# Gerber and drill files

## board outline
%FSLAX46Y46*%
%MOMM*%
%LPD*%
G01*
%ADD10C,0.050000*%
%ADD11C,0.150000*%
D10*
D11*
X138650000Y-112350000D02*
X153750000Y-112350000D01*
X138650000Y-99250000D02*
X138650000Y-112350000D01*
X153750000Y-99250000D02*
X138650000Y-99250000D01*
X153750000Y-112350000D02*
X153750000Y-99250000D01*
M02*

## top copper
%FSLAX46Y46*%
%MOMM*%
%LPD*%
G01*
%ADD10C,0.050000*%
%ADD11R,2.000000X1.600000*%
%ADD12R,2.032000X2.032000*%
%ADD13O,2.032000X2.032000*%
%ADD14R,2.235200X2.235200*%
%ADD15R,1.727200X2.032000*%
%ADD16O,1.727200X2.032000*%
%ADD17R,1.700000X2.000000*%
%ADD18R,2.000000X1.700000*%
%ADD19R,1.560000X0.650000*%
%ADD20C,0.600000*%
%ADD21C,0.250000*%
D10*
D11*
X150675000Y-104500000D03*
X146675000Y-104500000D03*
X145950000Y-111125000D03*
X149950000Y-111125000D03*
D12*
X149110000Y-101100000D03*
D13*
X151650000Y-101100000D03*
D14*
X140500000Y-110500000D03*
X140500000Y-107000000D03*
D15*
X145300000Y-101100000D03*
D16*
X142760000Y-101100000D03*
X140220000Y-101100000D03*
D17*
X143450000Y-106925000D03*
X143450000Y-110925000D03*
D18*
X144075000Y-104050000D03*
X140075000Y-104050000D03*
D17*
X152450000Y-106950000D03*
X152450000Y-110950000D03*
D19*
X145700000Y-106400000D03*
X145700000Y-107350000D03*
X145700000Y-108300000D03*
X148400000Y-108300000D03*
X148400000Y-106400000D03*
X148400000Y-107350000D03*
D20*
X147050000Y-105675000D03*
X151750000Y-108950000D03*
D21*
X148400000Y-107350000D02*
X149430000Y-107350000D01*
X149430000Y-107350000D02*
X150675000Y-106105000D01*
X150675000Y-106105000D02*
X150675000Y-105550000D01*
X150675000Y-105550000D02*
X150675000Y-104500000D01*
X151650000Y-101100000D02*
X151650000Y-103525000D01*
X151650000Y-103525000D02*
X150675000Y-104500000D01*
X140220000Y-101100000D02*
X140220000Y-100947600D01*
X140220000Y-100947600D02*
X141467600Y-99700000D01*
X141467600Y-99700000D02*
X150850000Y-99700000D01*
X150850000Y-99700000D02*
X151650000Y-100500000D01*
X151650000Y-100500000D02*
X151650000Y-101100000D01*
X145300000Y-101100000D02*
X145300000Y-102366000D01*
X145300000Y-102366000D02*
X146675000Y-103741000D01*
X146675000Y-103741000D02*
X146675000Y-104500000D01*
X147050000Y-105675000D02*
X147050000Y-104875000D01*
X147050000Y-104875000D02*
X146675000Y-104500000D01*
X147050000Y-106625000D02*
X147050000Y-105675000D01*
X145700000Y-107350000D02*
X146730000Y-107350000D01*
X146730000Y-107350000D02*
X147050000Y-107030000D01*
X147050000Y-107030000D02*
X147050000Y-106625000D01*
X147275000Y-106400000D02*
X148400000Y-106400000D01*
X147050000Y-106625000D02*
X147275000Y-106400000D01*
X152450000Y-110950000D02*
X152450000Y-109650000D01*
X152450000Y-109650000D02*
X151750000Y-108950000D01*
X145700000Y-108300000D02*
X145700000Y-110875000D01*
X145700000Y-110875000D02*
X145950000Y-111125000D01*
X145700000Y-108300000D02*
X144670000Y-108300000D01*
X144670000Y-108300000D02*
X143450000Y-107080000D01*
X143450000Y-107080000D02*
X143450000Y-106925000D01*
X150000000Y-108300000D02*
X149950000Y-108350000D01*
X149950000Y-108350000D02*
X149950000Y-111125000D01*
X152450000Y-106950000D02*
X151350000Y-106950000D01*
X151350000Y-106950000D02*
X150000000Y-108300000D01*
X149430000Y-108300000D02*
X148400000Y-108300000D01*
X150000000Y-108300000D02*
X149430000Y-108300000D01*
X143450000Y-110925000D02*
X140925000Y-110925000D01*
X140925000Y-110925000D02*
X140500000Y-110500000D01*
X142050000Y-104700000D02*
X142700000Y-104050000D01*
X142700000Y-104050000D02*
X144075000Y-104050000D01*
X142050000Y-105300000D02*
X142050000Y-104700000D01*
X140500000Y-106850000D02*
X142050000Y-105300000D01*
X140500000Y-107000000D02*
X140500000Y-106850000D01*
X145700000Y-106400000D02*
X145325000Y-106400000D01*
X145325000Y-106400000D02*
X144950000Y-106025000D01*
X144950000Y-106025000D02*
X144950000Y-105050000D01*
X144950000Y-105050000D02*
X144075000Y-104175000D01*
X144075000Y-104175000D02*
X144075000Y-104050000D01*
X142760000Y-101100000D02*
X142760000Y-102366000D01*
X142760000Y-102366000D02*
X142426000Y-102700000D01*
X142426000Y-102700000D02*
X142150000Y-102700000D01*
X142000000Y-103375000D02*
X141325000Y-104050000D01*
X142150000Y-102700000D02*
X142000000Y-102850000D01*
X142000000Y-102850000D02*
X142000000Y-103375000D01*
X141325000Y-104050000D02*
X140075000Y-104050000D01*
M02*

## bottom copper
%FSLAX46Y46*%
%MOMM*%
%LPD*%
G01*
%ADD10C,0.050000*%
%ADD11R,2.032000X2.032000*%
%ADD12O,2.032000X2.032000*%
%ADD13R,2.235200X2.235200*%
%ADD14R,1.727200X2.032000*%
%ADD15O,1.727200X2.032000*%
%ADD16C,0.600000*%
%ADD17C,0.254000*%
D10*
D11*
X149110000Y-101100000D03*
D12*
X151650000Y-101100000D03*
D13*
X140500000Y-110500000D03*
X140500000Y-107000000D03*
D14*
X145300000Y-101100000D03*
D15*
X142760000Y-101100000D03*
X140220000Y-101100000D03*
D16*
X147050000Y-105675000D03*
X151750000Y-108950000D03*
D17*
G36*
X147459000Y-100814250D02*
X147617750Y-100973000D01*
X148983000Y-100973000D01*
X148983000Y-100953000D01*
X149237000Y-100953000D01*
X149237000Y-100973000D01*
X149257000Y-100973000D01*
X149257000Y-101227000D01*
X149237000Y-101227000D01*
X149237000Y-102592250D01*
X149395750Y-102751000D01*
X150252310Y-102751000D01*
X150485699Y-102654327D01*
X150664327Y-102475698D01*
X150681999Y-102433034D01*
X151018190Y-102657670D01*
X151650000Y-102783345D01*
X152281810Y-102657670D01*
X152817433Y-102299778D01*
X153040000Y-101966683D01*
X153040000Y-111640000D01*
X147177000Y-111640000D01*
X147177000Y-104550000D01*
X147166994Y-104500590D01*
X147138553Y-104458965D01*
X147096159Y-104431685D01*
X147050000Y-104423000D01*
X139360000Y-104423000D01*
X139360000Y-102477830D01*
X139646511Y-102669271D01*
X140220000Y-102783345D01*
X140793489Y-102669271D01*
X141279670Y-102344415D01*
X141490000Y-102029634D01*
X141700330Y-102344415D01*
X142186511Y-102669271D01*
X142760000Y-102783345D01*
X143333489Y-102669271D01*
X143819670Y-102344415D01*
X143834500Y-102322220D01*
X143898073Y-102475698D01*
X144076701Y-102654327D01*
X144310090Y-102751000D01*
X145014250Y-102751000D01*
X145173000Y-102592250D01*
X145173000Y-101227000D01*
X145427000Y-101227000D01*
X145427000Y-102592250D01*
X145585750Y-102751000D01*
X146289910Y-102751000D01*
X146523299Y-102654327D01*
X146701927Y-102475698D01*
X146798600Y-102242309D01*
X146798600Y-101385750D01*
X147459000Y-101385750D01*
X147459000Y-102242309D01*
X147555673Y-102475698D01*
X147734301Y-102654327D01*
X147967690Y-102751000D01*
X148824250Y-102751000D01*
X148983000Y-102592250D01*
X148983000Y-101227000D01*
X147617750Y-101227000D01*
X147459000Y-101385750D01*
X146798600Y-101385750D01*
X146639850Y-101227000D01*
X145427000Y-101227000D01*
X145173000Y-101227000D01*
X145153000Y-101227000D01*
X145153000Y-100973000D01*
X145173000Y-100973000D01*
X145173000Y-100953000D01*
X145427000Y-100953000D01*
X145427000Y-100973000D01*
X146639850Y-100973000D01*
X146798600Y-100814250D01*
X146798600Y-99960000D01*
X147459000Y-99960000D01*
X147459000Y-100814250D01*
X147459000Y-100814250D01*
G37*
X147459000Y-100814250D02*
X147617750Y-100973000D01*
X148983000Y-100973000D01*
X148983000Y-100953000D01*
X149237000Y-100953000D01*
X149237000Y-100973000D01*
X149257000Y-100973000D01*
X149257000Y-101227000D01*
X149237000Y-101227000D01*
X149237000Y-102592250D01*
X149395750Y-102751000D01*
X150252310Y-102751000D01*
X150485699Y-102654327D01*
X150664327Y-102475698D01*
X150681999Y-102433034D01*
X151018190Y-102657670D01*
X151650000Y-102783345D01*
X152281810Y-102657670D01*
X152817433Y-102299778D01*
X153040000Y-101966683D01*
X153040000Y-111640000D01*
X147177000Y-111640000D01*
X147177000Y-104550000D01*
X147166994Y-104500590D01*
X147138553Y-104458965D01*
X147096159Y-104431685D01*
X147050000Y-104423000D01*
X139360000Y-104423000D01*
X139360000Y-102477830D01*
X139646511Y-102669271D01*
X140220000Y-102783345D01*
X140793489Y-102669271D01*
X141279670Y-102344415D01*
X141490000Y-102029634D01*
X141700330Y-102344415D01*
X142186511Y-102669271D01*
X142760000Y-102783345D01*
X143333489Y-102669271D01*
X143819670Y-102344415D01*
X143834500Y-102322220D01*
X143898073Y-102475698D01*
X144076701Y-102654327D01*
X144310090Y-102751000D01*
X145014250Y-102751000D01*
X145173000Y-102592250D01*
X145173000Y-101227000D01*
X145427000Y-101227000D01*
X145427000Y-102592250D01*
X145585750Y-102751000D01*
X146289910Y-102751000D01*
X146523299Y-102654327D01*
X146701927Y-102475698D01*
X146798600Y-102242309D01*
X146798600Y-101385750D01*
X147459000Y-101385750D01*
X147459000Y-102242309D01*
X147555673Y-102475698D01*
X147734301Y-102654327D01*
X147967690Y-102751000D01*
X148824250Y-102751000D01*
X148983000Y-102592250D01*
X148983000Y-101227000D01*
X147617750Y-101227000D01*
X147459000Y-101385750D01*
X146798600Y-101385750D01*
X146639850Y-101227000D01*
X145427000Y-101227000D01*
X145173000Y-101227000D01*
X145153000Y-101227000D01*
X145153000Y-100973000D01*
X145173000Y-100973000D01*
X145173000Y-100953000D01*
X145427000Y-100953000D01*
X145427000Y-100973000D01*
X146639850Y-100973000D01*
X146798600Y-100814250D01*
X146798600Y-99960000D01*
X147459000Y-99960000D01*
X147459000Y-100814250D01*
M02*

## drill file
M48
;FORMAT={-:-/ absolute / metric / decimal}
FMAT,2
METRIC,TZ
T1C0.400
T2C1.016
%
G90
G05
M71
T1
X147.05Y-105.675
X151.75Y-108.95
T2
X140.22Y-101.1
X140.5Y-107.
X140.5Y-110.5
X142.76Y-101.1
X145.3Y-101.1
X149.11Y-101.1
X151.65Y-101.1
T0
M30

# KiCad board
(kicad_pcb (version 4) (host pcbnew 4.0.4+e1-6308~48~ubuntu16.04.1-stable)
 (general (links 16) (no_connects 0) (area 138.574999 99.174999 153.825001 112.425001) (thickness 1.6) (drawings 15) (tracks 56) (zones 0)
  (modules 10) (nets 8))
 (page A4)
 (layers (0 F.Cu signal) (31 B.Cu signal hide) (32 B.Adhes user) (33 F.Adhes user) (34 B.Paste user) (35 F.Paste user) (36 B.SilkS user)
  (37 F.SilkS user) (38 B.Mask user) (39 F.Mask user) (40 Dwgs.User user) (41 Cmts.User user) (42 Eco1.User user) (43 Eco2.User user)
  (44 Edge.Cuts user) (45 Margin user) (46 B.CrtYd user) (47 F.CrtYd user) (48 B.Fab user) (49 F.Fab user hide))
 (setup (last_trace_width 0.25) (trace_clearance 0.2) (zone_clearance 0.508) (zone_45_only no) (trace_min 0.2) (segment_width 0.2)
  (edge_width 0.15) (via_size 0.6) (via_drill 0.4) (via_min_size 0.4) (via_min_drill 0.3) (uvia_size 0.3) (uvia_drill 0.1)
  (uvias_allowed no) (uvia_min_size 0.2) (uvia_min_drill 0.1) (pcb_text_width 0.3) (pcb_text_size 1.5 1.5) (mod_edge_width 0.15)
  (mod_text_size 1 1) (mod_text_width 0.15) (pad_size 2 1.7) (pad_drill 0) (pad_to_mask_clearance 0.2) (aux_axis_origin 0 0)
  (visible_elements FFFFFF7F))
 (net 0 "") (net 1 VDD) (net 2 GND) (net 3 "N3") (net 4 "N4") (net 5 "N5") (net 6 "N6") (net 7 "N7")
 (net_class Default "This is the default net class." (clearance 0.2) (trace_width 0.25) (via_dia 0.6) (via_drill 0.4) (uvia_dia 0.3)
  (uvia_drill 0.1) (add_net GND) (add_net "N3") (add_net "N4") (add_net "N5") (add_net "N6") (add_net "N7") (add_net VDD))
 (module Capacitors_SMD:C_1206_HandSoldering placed (layer F.Cu) (at 148.675 104.5 180)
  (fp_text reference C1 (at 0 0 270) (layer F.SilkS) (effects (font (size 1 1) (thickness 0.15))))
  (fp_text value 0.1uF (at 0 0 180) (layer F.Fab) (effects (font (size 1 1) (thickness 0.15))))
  (pad 1 smd rect (at -2 0 180) (size 2 1.6) (layers F.Cu F.Paste F.Mask) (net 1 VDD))
  (pad 2 smd rect (at 2 0 180) (size 2 1.6) (layers F.Cu F.Paste F.Mask) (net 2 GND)))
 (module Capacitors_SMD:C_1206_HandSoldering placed (layer F.Cu) (at 147.95 111.125)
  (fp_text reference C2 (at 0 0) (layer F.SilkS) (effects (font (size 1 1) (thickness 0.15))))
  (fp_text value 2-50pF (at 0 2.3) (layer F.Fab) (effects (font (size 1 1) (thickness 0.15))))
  (pad 1 smd rect (at -2 0) (size 2 1.6) (layers F.Cu F.Paste F.Mask) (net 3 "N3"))
  (pad 2 smd rect (at 2 0) (size 2 1.6) (layers F.Cu F.Paste F.Mask) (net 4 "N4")))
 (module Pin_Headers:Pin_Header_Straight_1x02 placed (layer F.Cu) (at 149.11 101.1 90)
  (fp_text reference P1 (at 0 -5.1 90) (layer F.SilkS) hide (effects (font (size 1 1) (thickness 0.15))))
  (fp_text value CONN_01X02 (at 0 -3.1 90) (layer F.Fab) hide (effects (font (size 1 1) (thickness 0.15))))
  (pad 1 thru_hole rect (at 0 0 90) (size 2.032 2.032) (drill 1.016) (layers *.Cu *.Mask F.SilkS) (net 2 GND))
  (pad 2 thru_hole oval (at 0 2.54 90) (size 2.032 2.032) (drill 1.016) (layers *.Cu *.Mask F.SilkS) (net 1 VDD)))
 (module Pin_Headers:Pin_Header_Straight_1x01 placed (layer F.Cu) (at 140.5 110.5 180)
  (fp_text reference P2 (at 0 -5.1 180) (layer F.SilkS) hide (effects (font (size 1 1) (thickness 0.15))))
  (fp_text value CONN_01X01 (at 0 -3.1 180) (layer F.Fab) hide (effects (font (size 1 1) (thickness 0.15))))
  (pad 1 thru_hole rect (at 0 0 180) (size 2.2352 2.2352) (drill 1.016) (layers *.Cu *.Mask F.SilkS) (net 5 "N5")))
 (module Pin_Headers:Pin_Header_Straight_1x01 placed (layer F.Cu) (at 140.5 107 90)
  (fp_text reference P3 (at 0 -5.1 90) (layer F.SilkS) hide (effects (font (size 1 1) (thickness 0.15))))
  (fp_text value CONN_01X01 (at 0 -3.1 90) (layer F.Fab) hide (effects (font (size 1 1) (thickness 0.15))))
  (pad 1 thru_hole rect (at 0 0 90) (size 2.2352 2.2352) (drill 1.016) (layers *.Cu *.Mask F.SilkS) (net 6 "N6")))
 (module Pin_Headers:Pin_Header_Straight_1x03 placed (layer F.Cu) (at 145.3 101.1 270)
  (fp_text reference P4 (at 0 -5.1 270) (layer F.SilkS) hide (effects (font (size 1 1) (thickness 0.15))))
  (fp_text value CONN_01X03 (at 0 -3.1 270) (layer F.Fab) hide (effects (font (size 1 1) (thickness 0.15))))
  (pad 1 thru_hole rect (at 0 0 270) (size 2.032 1.7272) (drill 1.016) (layers *.Cu *.Mask F.SilkS) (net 2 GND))
  (pad 2 thru_hole oval (at 0 2.54 270) (size 2.032 1.7272) (drill 1.016) (layers *.Cu *.Mask F.SilkS) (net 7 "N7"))
  (pad 3 thru_hole oval (at 0 5.08 270) (size 2.032 1.7272) (drill 1.016) (layers *.Cu *.Mask F.SilkS) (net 1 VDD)))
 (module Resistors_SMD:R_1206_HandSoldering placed (layer F.Cu) (at 143.45 108.925 270)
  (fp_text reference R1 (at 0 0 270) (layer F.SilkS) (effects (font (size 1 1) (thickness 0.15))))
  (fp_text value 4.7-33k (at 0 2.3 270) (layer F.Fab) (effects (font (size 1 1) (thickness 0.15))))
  (pad 1 smd rect (at -2 0 270) (size 2 1.7) (layers F.Cu F.Paste F.Mask) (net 3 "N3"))
  (pad 2 smd rect (at 2 0 270) (size 2 1.7) (layers F.Cu F.Paste F.Mask) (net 5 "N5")))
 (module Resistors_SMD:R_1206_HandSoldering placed (layer F.Cu) (at 142.075 104.05 180)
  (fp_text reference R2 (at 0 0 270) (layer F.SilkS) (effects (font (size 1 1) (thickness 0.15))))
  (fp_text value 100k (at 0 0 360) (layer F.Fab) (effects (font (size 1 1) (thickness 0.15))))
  (pad 1 smd rect (at -2 0 180) (size 2 1.7) (layers F.Cu F.Paste F.Mask) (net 6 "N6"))
  (pad 2 smd rect (at 2 0 180) (size 2 1.7) (layers F.Cu F.Paste F.Mask) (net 7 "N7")))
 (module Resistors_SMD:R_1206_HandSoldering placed (layer F.Cu) (at 152.45 108.95 270)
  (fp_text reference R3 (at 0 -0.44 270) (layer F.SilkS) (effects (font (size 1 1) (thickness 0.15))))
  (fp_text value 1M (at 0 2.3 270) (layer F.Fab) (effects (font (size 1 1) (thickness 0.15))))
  (pad 1 smd rect (at -2 0 270) (size 2 1.7) (layers F.Cu F.Paste F.Mask) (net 4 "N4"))
  (pad 2 smd rect (at 2 0 270) (size 2 1.7) (layers F.Cu F.Paste F.Mask) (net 2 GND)))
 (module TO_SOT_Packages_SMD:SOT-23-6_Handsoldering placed (layer F.Cu) (at 147.05 107.35)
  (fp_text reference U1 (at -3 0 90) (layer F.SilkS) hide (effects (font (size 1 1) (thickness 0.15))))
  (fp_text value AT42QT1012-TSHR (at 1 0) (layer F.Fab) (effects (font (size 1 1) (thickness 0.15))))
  (pad 1 smd rect (at -1.35 -0.95) (size 1.56 0.65) (layers F.Cu F.Paste F.Mask) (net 6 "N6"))
  (pad 2 smd rect (at -1.35 0) (size 1.56 0.65) (layers F.Cu F.Paste F.Mask) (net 2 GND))
  (pad 3 smd rect (at -1.35 0.95) (size 1.56 0.65) (layers F.Cu F.Paste F.Mask) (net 3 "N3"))
  (pad 4 smd rect (at 1.35 0.95) (size 1.56 0.65) (layers F.Cu F.Paste F.Mask) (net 4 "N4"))
  (pad 6 smd rect (at 1.35 -0.95) (size 1.56 0.65) (layers F.Cu F.Paste F.Mask) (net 2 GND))
  (pad 5 smd rect (at 1.35 0) (size 1.56 0.65) (layers F.Cu F.Paste F.Mask) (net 1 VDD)))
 (gr_line (start 138.65 112.35) (end 153.75 112.35) (layer Edge.Cuts) (width 0.15))
 (gr_line (start 138.65 99.25) (end 138.65 112.35) (layer Edge.Cuts) (width 0.15))
 (gr_line (start 153.75 99.25) (end 138.65 99.25) (layer Edge.Cuts) (width 0.15))
 (gr_line (start 153.75 112.35) (end 153.75 99.25) (layer Edge.Cuts) (width 0.15))
 (segment (start 148.4 107.35) (end 149.43 107.35) (width 0.25) (layer F.Cu) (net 1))
 (segment (start 149.43 107.35) (end 150.675 106.105) (width 0.25) (layer F.Cu) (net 1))
 (segment (start 150.675 106.105) (end 150.675 105.55) (width 0.25) (layer F.Cu) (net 1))
 (segment (start 150.675 105.55) (end 150.675 104.5) (width 0.25) (layer F.Cu) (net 1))
 (segment (start 151.65 101.1) (end 151.65 103.525) (width 0.25) (layer F.Cu) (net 1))
 (segment (start 151.65 103.525) (end 150.675 104.5) (width 0.25) (layer F.Cu) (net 1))
 (segment (start 140.22 101.1) (end 140.22 100.9476) (width 0.25) (layer F.Cu) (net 1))
 (segment (start 140.22 100.9476) (end 141.4676 99.7) (width 0.25) (layer F.Cu) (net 1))
 (segment (start 141.4676 99.7) (end 150.85 99.7) (width 0.25) (layer F.Cu) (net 1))
 (segment (start 150.85 99.7) (end 151.65 100.5) (width 0.25) (layer F.Cu) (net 1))
 (segment (start 151.65 100.5) (end 151.65 101.1) (width 0.25) (layer F.Cu) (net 1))
 (segment (start 145.3 101.1) (end 145.3 102.366) (width 0.25) (layer F.Cu) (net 2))
 (segment (start 145.3 102.366) (end 146.675 103.741) (width 0.25) (layer F.Cu) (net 2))
 (segment (start 146.675 103.741) (end 146.675 104.5) (width 0.25) (layer F.Cu) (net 2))
 (segment (start 147.05 105.675) (end 147.05 104.875) (width 0.25) (layer F.Cu) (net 2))
 (segment (start 147.05 104.875) (end 146.675 104.5) (width 0.25) (layer F.Cu) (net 2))
 (via (at 147.05 105.675) (size 0.6) (drill 0.4) (layers F.Cu B.Cu) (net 2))
 (segment (start 147.05 106.625) (end 147.05 105.675) (width 0.25) (layer F.Cu) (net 2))
 (segment (start 145.7 107.35) (end 146.73 107.35) (width 0.25) (layer F.Cu) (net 2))
 (segment (start 146.73 107.35) (end 147.05 107.03) (width 0.25) (layer F.Cu) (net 2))
 (segment (start 147.05 107.03) (end 147.05 106.625) (width 0.25) (layer F.Cu) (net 2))
 (segment (start 147.275 106.4) (end 148.4 106.4) (width 0.25) (layer F.Cu) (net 2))
 (segment (start 147.05 106.625) (end 147.275 106.4) (width 0.25) (layer F.Cu) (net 2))
 (segment (start 152.45 110.95) (end 152.45 109.65) (width 0.25) (layer F.Cu) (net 2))
 (segment (start 152.45 109.65) (end 151.75 108.95) (width 0.25) (layer F.Cu) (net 2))
 (via (at 151.75 108.95) (size 0.6) (drill 0.4) (layers F.Cu B.Cu) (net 2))
 (segment (start 145.7 108.3) (end 145.7 110.875) (width 0.25) (layer F.Cu) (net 3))
 (segment (start 145.7 110.875) (end 145.95 111.125) (width 0.25) (layer F.Cu) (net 3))
 (segment (start 145.7 108.3) (end 144.67 108.3) (width 0.25) (layer F.Cu) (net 3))
 (segment (start 144.67 108.3) (end 143.45 107.08) (width 0.25) (layer F.Cu) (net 3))
 (segment (start 143.45 107.08) (end 143.45 106.925) (width 0.25) (layer F.Cu) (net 3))
 (segment (start 150 108.3) (end 149.95 108.35) (width 0.25) (layer F.Cu) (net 4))
 (segment (start 149.95 108.35) (end 149.95 111.125) (width 0.25) (layer F.Cu) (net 4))
 (segment (start 152.45 106.95) (end 151.35 106.95) (width 0.25) (layer F.Cu) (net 4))
 (segment (start 151.35 106.95) (end 150 108.3) (width 0.25) (layer F.Cu) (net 4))
 (segment (start 149.43 108.3) (end 148.4 108.3) (width 0.25) (layer F.Cu) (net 4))
 (segment (start 150 108.3) (end 149.43 108.3) (width 0.25) (layer F.Cu) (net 4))
 (segment (start 143.45 110.925) (end 140.925 110.925) (width 0.25) (layer F.Cu) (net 5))
 (segment (start 140.925 110.925) (end 140.5 110.5) (width 0.25) (layer F.Cu) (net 5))
 (segment (start 142.05 104.7) (end 142.7 104.05) (width 0.25) (layer F.Cu) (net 6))
 (segment (start 142.7 104.05) (end 144.075 104.05) (width 0.25) (layer F.Cu) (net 6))
 (segment (start 142.05 105.3) (end 142.05 104.7) (width 0.25) (layer F.Cu) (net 6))
 (segment (start 140.5 106.85) (end 142.05 105.3) (width 0.25) (layer F.Cu) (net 6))
 (segment (start 140.5 107) (end 140.5 106.85) (width 0.25) (layer F.Cu) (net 6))
 (segment (start 145.7 106.4) (end 145.325 106.4) (width 0.25) (layer F.Cu) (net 6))
 (segment (start 145.325 106.4) (end 144.95 106.025) (width 0.25) (layer F.Cu) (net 6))
 (segment (start 144.95 106.025) (end 144.95 105.05) (width 0.25) (layer F.Cu) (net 6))
 (segment (start 144.95 105.05) (end 144.075 104.175) (width 0.25) (layer F.Cu) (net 6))
 (segment (start 144.075 104.175) (end 144.075 104.05) (width 0.25) (layer F.Cu) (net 6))
 (segment (start 142.76 101.1) (end 142.76 102.366) (width 0.25) (layer F.Cu) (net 7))
 (segment (start 142.76 102.366) (end 142.426 102.7) (width 0.25) (layer F.Cu) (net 7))
 (segment (start 142.426 102.7) (end 142.15 102.7) (width 0.25) (layer F.Cu) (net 7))
 (segment (start 142 103.375) (end 141.325 104.05) (width 0.25) (layer F.Cu) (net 7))
 (segment (start 142.15 102.7) (end 142 102.85) (width 0.25) (layer F.Cu) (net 7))
 (segment (start 142 102.85) (end 142 103.375) (width 0.25) (layer F.Cu) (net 7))
 (segment (start 141.325 104.05) (end 140.075 104.05) (width 0.25) (layer F.Cu) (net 7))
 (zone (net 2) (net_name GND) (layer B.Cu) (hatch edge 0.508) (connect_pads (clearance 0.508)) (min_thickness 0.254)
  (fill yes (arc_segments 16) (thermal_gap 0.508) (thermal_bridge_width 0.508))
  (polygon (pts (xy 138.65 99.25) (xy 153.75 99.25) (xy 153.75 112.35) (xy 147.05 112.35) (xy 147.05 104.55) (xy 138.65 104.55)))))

